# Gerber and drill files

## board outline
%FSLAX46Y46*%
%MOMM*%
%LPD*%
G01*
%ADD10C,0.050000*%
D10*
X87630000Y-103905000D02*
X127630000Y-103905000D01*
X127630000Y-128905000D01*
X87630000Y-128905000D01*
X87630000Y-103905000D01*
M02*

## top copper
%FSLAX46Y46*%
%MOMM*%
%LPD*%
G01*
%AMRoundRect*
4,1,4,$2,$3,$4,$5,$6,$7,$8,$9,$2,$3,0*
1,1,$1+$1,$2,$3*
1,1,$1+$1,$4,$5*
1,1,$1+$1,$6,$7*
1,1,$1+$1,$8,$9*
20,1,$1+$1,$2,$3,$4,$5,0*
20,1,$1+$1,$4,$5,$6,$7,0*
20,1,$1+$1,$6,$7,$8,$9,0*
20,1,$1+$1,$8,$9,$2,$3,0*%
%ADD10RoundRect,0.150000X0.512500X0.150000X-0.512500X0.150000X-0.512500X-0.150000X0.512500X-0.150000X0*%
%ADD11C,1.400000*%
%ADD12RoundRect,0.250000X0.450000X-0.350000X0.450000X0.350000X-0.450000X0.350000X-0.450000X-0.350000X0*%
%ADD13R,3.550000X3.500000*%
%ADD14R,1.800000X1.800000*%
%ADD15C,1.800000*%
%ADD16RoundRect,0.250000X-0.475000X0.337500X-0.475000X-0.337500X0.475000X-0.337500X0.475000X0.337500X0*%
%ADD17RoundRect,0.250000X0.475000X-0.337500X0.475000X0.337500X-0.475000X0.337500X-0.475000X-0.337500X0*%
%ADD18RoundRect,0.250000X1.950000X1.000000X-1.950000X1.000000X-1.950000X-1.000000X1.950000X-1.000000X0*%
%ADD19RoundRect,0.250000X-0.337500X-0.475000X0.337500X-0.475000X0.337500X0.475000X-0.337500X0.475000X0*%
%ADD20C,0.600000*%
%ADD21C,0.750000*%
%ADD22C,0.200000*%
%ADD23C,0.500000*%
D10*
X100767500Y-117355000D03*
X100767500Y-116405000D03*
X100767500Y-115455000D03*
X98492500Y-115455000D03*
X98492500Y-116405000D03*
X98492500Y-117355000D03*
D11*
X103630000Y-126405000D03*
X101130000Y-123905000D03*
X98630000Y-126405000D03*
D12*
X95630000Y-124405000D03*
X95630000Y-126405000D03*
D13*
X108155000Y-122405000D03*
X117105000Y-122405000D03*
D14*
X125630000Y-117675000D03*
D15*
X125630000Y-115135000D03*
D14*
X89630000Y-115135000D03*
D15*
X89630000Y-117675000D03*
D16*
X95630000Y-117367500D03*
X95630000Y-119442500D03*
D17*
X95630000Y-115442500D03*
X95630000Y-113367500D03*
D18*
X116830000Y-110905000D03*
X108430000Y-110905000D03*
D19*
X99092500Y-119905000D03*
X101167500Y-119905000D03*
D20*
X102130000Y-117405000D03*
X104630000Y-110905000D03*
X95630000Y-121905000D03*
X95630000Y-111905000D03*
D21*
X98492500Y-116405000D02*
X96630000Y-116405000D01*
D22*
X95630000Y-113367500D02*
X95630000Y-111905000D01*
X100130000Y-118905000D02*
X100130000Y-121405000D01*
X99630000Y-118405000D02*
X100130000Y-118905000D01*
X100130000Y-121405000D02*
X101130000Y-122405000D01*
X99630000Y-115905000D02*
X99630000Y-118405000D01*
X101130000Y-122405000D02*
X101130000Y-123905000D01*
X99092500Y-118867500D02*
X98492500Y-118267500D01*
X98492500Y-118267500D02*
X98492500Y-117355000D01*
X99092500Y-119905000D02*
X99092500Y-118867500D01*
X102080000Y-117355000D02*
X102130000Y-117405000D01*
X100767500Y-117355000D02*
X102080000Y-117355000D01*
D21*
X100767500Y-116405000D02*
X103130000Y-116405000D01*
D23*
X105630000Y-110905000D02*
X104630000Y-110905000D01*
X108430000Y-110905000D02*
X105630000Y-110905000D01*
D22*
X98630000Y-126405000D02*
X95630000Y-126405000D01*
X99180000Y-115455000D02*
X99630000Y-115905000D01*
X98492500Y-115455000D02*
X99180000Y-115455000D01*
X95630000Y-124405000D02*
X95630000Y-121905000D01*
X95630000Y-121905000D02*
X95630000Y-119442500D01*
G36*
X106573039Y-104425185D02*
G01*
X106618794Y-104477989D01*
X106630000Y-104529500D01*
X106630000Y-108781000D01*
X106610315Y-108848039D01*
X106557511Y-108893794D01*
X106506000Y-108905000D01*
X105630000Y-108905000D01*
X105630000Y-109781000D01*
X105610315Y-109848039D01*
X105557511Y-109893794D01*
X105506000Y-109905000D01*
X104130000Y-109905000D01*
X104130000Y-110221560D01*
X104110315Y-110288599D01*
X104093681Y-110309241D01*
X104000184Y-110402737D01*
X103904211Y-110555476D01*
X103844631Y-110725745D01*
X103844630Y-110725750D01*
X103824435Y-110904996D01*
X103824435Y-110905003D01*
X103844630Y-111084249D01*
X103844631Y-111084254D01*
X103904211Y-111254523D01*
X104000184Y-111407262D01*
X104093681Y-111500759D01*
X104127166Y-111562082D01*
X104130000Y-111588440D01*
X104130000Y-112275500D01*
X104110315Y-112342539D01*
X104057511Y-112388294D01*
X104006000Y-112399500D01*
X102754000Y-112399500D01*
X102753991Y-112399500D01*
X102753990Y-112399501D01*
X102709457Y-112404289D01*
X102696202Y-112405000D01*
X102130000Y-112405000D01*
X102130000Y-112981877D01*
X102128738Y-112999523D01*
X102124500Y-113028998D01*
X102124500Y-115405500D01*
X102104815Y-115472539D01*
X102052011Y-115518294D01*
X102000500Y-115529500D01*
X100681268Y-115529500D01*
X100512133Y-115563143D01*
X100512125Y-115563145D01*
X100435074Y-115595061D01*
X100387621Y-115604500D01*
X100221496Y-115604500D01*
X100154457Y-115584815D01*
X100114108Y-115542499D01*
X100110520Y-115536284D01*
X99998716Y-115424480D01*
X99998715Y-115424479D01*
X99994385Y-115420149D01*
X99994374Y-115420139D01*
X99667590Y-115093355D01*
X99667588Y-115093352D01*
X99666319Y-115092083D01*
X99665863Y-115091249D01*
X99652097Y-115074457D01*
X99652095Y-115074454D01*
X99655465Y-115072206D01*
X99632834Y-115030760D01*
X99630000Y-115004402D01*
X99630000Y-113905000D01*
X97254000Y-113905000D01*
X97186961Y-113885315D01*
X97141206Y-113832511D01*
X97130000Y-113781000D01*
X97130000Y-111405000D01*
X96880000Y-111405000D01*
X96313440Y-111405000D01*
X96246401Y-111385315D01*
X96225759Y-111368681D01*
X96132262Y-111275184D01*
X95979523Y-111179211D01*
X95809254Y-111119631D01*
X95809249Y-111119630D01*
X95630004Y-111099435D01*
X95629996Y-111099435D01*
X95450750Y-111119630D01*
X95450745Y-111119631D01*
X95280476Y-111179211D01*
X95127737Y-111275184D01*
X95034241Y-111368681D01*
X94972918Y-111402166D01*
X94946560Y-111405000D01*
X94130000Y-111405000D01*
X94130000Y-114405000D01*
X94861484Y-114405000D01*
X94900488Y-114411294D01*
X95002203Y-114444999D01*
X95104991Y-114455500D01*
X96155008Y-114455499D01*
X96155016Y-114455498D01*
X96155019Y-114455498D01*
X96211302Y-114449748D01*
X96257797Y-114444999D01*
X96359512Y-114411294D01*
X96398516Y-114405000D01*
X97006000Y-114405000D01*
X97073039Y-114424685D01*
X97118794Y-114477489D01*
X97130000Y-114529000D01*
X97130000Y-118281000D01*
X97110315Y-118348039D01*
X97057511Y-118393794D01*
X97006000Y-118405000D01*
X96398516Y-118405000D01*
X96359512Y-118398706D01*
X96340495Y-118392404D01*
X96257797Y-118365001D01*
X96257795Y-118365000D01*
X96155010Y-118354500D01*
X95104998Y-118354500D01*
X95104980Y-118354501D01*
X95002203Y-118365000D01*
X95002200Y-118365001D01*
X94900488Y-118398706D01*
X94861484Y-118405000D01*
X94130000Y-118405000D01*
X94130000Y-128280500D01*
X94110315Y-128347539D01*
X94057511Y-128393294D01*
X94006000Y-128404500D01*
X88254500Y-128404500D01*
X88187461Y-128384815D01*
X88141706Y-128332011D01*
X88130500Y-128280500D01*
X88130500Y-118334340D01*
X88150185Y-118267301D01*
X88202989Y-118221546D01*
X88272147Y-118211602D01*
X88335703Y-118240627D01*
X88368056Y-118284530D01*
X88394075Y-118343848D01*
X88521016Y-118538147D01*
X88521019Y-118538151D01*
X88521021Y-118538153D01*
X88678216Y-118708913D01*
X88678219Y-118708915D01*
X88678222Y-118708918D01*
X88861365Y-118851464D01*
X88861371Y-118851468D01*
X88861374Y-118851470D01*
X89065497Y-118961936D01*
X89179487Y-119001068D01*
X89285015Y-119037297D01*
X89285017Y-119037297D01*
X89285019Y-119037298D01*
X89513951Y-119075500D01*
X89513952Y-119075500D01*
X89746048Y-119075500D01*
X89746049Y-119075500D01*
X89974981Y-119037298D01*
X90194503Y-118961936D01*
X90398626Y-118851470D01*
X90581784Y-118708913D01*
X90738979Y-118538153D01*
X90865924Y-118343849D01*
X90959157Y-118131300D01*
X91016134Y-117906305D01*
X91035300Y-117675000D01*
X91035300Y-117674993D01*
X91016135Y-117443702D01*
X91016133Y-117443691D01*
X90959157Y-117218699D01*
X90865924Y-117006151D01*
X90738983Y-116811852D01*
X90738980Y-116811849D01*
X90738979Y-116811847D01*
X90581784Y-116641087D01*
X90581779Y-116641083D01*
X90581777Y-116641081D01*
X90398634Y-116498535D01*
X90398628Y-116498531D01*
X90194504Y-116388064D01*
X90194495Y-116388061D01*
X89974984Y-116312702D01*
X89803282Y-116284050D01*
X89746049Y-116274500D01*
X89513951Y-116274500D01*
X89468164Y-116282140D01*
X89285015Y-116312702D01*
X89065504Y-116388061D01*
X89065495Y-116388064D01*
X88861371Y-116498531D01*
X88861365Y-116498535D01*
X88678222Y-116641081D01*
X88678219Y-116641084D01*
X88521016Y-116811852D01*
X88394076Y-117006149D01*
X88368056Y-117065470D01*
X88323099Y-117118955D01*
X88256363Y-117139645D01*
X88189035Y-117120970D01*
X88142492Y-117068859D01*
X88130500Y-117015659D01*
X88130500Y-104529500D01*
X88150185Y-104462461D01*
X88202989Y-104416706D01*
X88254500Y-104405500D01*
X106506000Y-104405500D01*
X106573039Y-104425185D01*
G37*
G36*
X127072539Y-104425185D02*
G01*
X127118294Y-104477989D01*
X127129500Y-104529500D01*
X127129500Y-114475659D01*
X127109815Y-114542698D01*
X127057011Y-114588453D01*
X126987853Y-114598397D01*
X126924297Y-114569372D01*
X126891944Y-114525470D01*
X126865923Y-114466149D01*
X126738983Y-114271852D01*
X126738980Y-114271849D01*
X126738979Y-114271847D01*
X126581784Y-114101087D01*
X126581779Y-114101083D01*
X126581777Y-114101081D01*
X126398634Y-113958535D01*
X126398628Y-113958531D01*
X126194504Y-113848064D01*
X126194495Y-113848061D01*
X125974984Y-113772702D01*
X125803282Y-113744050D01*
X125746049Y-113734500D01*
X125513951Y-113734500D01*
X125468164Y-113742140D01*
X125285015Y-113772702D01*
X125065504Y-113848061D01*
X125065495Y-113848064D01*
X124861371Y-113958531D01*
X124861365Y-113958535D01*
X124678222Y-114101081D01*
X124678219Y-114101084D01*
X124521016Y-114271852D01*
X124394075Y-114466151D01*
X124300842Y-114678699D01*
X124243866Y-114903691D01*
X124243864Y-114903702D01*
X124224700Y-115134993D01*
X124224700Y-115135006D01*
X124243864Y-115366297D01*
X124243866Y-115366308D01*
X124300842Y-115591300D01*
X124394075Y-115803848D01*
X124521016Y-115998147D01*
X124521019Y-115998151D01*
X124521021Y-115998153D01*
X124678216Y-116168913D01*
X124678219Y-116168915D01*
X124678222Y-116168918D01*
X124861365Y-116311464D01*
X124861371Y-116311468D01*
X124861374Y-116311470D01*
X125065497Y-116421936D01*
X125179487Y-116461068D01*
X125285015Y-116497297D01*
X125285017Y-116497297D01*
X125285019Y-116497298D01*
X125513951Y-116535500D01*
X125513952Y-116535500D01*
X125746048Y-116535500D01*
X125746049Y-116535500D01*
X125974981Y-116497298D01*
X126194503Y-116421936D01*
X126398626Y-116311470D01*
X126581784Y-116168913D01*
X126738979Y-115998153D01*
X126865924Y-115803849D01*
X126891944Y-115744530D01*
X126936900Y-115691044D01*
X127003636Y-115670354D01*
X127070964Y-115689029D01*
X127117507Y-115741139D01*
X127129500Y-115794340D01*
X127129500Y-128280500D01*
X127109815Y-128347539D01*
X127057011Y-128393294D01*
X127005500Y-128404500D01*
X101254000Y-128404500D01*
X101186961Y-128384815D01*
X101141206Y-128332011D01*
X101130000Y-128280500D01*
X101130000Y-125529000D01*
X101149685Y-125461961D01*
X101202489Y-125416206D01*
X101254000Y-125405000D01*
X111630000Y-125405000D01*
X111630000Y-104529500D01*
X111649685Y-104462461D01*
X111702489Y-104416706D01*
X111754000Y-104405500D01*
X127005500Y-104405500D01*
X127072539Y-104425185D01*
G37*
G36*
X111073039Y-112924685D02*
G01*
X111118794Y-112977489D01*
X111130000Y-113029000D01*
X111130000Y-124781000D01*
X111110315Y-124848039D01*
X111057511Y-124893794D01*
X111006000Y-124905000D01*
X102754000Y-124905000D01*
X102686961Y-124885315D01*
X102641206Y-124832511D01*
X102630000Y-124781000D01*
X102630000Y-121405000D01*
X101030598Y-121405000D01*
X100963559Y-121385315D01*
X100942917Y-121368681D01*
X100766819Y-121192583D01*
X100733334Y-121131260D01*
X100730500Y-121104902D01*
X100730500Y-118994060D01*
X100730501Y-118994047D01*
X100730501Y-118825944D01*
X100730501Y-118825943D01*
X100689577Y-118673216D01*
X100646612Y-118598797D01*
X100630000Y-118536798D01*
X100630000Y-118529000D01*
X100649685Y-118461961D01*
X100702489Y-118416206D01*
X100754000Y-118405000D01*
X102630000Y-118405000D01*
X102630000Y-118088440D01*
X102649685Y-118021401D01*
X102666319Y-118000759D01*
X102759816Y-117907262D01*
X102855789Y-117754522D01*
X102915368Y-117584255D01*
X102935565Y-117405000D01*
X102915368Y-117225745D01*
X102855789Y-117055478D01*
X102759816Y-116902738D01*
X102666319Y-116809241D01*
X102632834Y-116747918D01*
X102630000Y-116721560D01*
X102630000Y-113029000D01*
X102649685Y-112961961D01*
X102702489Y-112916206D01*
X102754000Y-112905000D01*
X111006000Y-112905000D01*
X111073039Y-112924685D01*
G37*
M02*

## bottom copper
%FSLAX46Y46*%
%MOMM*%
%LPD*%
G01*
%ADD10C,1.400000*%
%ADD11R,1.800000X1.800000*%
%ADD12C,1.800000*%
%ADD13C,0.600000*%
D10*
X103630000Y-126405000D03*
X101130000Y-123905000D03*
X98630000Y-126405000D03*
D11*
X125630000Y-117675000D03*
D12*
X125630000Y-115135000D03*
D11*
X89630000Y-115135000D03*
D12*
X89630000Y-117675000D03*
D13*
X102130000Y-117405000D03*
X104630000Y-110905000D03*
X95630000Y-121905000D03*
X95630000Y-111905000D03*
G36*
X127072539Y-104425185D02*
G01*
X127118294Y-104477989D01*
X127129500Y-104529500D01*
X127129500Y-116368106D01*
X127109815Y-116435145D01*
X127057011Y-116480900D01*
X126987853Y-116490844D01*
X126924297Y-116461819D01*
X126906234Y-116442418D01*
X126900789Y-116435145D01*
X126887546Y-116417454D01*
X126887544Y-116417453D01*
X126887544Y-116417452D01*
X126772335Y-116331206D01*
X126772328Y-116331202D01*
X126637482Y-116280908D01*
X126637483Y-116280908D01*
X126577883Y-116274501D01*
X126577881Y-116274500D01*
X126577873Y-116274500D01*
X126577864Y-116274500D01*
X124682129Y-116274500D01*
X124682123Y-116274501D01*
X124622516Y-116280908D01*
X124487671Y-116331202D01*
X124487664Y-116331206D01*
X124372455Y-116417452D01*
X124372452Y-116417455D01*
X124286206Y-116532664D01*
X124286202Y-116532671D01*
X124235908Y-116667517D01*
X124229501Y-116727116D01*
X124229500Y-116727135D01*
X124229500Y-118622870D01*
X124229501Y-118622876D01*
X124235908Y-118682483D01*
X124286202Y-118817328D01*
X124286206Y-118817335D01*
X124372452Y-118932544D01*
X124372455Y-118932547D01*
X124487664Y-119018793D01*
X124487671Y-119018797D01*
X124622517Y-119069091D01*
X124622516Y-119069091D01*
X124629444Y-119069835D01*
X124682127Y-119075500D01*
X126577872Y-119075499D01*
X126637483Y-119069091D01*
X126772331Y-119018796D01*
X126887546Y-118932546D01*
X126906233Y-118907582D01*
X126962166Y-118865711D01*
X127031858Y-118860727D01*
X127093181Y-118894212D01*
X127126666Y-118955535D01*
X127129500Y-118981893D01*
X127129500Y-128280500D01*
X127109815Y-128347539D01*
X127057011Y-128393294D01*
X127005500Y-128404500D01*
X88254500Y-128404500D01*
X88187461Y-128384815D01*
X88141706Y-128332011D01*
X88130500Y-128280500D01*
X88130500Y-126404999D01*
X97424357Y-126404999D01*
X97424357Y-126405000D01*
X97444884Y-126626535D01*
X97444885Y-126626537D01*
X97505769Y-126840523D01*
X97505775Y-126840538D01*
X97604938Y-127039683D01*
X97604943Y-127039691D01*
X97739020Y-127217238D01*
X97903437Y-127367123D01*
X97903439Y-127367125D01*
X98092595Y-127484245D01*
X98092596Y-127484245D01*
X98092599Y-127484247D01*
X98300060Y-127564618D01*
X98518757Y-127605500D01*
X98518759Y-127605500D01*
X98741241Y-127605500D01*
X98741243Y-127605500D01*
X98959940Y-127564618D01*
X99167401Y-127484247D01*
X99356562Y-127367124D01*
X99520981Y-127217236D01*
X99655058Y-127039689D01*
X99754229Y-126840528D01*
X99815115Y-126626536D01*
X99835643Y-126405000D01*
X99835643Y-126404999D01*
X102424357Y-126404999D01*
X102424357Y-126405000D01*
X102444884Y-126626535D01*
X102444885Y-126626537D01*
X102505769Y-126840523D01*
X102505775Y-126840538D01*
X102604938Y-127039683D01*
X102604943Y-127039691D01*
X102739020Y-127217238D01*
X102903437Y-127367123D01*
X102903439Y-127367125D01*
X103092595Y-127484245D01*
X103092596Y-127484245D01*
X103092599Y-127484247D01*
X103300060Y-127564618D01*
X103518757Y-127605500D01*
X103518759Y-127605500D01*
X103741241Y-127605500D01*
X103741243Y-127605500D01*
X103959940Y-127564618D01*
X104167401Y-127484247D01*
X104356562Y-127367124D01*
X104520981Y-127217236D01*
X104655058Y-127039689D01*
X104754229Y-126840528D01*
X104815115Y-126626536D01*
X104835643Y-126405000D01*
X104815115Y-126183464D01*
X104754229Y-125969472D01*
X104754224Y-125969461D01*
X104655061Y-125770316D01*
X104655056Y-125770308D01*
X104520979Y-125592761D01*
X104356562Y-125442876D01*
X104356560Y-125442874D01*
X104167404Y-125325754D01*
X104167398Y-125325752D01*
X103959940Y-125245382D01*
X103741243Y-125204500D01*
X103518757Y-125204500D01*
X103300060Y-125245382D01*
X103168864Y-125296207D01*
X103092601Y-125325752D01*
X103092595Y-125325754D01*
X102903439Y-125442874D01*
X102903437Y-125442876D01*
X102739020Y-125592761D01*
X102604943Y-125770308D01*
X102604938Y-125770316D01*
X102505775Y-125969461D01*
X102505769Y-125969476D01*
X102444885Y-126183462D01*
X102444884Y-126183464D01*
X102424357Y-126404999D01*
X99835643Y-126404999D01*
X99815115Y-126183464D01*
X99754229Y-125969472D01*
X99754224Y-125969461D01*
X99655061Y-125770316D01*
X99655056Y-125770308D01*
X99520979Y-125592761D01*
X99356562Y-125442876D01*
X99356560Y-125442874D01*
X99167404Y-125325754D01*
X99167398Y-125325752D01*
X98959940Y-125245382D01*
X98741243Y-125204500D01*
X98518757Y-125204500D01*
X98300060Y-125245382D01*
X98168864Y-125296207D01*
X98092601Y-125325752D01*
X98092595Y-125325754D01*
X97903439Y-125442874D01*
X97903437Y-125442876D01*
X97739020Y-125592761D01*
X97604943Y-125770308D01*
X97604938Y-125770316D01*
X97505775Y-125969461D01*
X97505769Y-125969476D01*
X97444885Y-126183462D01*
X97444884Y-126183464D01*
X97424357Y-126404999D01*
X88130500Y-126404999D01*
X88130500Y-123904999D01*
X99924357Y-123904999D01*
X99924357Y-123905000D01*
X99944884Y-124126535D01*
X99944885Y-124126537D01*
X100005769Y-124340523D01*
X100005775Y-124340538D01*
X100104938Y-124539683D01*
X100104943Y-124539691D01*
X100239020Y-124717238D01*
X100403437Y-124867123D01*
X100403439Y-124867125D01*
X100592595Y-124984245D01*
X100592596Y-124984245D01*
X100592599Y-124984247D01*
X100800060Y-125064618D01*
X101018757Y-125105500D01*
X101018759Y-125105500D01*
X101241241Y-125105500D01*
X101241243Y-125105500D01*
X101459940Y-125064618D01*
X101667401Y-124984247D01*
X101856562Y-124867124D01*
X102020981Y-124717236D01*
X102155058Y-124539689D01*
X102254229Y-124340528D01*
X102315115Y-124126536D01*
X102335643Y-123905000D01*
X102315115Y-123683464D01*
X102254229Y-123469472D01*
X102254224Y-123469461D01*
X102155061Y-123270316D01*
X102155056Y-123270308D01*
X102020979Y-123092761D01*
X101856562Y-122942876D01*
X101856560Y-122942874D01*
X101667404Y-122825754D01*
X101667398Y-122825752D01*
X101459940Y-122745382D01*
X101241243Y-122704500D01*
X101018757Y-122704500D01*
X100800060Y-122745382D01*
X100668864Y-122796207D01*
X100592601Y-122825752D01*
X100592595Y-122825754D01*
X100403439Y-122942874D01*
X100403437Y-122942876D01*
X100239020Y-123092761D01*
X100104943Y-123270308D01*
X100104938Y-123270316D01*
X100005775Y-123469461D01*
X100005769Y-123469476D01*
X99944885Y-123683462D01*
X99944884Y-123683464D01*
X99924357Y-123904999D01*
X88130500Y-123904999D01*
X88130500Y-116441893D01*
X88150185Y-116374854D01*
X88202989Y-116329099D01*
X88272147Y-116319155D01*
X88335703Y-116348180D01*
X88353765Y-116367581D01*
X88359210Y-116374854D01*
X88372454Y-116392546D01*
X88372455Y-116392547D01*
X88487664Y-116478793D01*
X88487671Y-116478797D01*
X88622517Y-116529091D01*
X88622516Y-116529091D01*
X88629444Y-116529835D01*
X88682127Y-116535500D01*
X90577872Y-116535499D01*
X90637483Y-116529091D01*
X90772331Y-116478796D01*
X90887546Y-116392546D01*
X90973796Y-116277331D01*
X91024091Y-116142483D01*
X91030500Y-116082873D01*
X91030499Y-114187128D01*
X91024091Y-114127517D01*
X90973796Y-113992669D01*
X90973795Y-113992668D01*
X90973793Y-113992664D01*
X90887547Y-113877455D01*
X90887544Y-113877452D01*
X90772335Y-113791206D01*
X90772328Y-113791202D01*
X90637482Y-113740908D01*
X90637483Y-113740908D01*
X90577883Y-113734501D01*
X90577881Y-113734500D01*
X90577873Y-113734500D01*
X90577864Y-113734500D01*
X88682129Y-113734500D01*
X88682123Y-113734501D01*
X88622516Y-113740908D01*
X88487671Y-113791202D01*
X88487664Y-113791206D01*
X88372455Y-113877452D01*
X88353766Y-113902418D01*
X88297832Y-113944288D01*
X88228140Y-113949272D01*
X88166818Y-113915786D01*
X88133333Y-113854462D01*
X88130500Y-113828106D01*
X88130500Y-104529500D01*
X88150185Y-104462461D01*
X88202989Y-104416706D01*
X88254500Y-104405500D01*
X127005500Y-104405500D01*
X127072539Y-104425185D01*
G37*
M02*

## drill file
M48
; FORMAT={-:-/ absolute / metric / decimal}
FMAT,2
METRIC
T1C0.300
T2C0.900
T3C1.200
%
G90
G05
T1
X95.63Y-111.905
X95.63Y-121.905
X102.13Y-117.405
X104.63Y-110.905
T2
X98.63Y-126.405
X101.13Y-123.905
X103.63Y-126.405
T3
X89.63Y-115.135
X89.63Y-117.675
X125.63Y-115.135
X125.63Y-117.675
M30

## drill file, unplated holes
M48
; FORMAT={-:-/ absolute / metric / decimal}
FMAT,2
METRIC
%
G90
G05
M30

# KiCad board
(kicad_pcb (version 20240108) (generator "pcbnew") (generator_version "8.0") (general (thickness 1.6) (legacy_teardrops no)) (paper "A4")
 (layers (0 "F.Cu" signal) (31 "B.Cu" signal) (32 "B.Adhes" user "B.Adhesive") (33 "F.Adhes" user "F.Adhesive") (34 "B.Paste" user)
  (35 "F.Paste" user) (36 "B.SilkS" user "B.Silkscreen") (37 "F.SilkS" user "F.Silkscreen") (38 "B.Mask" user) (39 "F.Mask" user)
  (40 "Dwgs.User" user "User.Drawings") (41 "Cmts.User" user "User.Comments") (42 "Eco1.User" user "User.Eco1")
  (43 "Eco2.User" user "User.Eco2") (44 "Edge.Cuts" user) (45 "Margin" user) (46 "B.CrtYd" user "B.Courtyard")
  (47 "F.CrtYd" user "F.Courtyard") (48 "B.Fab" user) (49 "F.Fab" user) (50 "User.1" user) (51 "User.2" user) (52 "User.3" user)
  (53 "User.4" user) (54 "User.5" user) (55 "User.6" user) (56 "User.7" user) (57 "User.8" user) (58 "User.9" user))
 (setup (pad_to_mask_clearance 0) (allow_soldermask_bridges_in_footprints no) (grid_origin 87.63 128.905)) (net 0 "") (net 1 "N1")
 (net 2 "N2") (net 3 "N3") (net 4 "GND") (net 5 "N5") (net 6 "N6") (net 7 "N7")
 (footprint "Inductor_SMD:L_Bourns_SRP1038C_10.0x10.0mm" (layer "F.Cu") (at 112.63 122.405)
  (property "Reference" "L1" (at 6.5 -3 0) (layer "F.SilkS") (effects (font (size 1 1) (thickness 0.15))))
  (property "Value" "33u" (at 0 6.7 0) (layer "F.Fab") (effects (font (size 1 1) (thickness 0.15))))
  (pad "1" smd rect (at -4.475 0) (size 3.55 3.5) (layers "F.Cu" "F.Paste" "F.Mask") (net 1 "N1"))
  (pad "2" smd rect (at 4.475 0) (size 3.55 3.5) (layers "F.Cu" "F.Paste" "F.Mask") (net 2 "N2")))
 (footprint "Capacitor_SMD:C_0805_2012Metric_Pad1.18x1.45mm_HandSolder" (layer "F.Cu") (at 95.63 118.405 -90)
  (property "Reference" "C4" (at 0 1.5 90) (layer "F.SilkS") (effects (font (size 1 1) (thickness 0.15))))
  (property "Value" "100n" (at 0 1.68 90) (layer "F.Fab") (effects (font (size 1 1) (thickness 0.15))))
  (pad "1" smd roundrect (at -1.0375 0 270) (size 1.175 1.45) (layers "F.Cu" "F.Paste" "F.Mask") (roundrect_rratio 0.212766) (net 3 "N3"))
  (pad "2" smd roundrect (at 1.0375 0 270) (size 1.175 1.45) (layers "F.Cu" "F.Paste" "F.Mask") (roundrect_rratio 0.212766) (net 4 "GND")))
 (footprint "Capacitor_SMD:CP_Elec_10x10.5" (layer "F.Cu") (at 112.63 110.905 180)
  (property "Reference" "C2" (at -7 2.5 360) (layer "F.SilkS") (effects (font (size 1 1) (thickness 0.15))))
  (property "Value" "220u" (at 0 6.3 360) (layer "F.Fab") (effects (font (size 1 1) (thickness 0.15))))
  (pad "1" smd roundrect (at -4.2 0 180) (size 4.4 2.5) (layers "F.Cu" "F.Paste" "F.Mask") (roundrect_rratio 0.1) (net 2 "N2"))
  (pad "2" smd roundrect (at 4.2 0 180) (size 4.4 2.5) (layers "F.Cu" "F.Paste" "F.Mask") (roundrect_rratio 0.1) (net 4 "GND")))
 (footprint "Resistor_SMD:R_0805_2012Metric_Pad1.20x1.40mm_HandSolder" (layer "F.Cu") (at 95.63 125.405 90)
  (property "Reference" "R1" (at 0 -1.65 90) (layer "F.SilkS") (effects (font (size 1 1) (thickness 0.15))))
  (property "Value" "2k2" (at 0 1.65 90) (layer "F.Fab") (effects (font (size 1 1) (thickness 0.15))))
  (pad "1" smd roundrect (at -1 0 90) (size 1.2 1.4) (layers "F.Cu" "F.Paste" "F.Mask") (roundrect_rratio 0.208333) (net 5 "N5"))
  (pad "2" smd roundrect (at 1 0 90) (size 1.2 1.4) (layers "F.Cu" "F.Paste" "F.Mask") (roundrect_rratio 0.208333) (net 4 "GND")))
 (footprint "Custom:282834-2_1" (layer "F.Cu") (at 89.63 115.135 -90)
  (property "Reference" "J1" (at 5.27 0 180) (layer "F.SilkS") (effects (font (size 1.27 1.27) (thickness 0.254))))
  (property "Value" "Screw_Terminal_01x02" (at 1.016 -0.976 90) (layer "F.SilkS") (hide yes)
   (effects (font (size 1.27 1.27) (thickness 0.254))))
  (pad "1" thru_hole rect (at 0 0 270) (size 1.8 1.8) (drill 1.2) (layers "*.Cu" "*.Mask") (remove_unused_layers no) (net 3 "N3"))
  (pad "2" thru_hole circle (at 2.54 0 270) (size 1.8 1.8) (drill 1.2) (layers "*.Cu" "*.Mask") (remove_unused_layers no) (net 4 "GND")))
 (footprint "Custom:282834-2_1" (layer "F.Cu") (at 125.63 117.675 90)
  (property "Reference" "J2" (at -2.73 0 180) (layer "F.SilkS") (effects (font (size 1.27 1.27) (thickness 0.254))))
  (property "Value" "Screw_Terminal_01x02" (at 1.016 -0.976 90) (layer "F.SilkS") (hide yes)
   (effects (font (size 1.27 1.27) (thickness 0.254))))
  (pad "1" thru_hole rect (at 0 0 90) (size 1.8 1.8) (drill 1.2) (layers "*.Cu" "*.Mask") (remove_unused_layers no) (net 2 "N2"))
  (pad "2" thru_hole circle (at 2.54 0 90) (size 1.8 1.8) (drill 1.2) (layers "*.Cu" "*.Mask") (remove_unused_layers no) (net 4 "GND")))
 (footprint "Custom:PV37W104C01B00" (layer "F.Cu") (at 98.63 126.405)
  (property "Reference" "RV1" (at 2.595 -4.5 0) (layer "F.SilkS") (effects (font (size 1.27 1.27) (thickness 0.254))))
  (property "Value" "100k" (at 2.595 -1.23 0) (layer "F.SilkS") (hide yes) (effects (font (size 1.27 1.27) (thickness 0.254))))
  (pad "1" thru_hole circle (at 0 0) (size 1.4 1.4) (drill 0.9) (layers "*.Cu" "*.Mask") (remove_unused_layers no) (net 5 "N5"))
  (pad "2" thru_hole circle (at 2.5 -2.5) (size 1.4 1.4) (drill 0.9) (layers "*.Cu" "*.Mask") (remove_unused_layers no) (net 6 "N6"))
  (pad "3" thru_hole circle (at 5 0) (size 1.4 1.4) (drill 0.9) (layers "*.Cu" "*.Mask") (remove_unused_layers no) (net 2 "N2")))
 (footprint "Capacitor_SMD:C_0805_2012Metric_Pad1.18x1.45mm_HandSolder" (layer "F.Cu") (at 100.13 119.905)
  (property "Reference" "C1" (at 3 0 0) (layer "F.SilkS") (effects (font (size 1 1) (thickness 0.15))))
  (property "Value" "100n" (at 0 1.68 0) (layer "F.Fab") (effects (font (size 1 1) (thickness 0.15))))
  (pad "1" smd roundrect (at -1.0375 0) (size 1.175 1.45) (layers "F.Cu" "F.Paste" "F.Mask") (roundrect_rratio 0.212766) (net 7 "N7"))
  (pad "2" smd roundrect (at 1.0375 0) (size 1.175 1.45) (layers "F.Cu" "F.Paste" "F.Mask") (roundrect_rratio 0.212766) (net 1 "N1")))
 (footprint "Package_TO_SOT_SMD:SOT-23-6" (layer "F.Cu") (at 99.63 116.405 180)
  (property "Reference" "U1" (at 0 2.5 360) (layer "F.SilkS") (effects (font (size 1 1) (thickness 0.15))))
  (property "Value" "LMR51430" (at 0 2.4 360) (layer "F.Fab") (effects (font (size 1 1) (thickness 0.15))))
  (pad "1" smd roundrect (at -1.1375 -0.95 180) (size 1.325 0.6) (layers "F.Cu" "F.Paste" "F.Mask") (roundrect_rratio 0.25) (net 4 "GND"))
  (pad "2" smd roundrect (at -1.1375 0 180) (size 1.325 0.6) (layers "F.Cu" "F.Paste" "F.Mask") (roundrect_rratio 0.25) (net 1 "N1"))
  (pad "3" smd roundrect (at -1.1375 0.95 180) (size 1.325 0.6) (layers "F.Cu" "F.Paste" "F.Mask") (roundrect_rratio 0.25) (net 3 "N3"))
  (pad "4" smd roundrect (at 1.1375 0.95 180) (size 1.325 0.6) (layers "F.Cu" "F.Paste" "F.Mask") (roundrect_rratio 0.25) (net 6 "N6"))
  (pad "5" smd roundrect (at 1.1375 0 180) (size 1.325 0.6) (layers "F.Cu" "F.Paste" "F.Mask") (roundrect_rratio 0.25) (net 3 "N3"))
  (pad "6" smd roundrect (at 1.1375 -0.95 180) (size 1.325 0.6) (layers "F.Cu" "F.Paste" "F.Mask") (roundrect_rratio 0.25) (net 7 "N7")))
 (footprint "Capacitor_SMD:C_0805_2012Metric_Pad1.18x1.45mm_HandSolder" (layer "F.Cu") (at 95.63 114.405 90)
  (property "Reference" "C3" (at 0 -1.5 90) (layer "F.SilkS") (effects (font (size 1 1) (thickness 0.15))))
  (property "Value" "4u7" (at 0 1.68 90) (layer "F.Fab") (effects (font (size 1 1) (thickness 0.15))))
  (pad "1" smd roundrect (at -1.0375 0 90) (size 1.175 1.45) (layers "F.Cu" "F.Paste" "F.Mask") (roundrect_rratio 0.212766) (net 3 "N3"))
  (pad "2" smd roundrect (at 1.0375 0 90) (size 1.175 1.45) (layers "F.Cu" "F.Paste" "F.Mask") (roundrect_rratio 0.212766) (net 4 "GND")))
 (gr_rect (start 87.63 103.905) (end 127.63 128.905) (stroke (width 0.05) (type default)) (fill none) (layer "Edge.Cuts"))
 (segment (start 99.0925 118.8675) (end 98.4925 118.2675) (width 0.2) (layer "F.Cu") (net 7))
 (segment (start 98.4925 118.2675) (end 98.4925 117.355) (width 0.2) (layer "F.Cu") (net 7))
 (segment (start 99.0925 119.905) (end 99.0925 118.8675) (width 0.2) (layer "F.Cu") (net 7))
 (segment (start 100.7675 116.405) (end 103.13 116.405) (width 0.75) (layer "F.Cu") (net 1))
 (segment (start 108.43 110.905) (end 105.63 110.905) (width 0.5) (layer "F.Cu") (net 4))
 (segment (start 95.63 121.905) (end 95.63 119.4425) (width 0.2) (layer "F.Cu") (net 4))
 (segment (start 102.08 117.355) (end 102.13 117.405) (width 0.2) (layer "F.Cu") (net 4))
 (segment (start 95.63 113.3675) (end 95.63 111.905) (width 0.2) (layer "F.Cu") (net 4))
 (segment (start 100.7675 117.355) (end 102.08 117.355) (width 0.2) (layer "F.Cu") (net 4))
 (segment (start 105.63 110.905) (end 104.63 110.905) (width 0.5) (layer "F.Cu") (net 4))
 (segment (start 95.63 124.405) (end 95.63 121.905) (width 0.2) (layer "F.Cu") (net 4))
 (via (at 95.63 111.905) (size 0.6) (drill 0.3) (layers "F.Cu" "B.Cu") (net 4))
 (via (at 104.63 110.905) (size 0.6) (drill 0.3) (layers "F.Cu" "B.Cu") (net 4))
 (via (at 95.63 121.905) (size 0.6) (drill 0.3) (layers "F.Cu" "B.Cu") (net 4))
 (via (at 102.13 117.405) (size 0.6) (drill 0.3) (layers "F.Cu" "B.Cu") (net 4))
 (segment (start 98.4925 116.405) (end 96.63 116.405) (width 0.75) (layer "F.Cu") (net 3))
 (segment (start 98.63 126.405) (end 95.63 126.405) (width 0.2) (layer "F.Cu") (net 5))
 (segment (start 99.63 118.405) (end 100.13 118.905) (width 0.2) (layer "F.Cu") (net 6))
 (segment (start 100.13 121.405) (end 101.13 122.405) (width 0.2) (layer "F.Cu") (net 6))
 (segment (start 98.4925 115.455) (end 99.18 115.455) (width 0.2) (layer "F.Cu") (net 6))
 (segment (start 99.18 115.455) (end 99.63 115.905) (width 0.2) (layer "F.Cu") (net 6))
 (segment (start 101.13 122.405) (end 101.13 123.905) (width 0.2) (layer "F.Cu") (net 6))
 (segment (start 99.63 115.905) (end 99.63 118.405) (width 0.2) (layer "F.Cu") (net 6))
 (segment (start 100.13 118.905) (end 100.13 121.405) (width 0.2) (layer "F.Cu") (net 6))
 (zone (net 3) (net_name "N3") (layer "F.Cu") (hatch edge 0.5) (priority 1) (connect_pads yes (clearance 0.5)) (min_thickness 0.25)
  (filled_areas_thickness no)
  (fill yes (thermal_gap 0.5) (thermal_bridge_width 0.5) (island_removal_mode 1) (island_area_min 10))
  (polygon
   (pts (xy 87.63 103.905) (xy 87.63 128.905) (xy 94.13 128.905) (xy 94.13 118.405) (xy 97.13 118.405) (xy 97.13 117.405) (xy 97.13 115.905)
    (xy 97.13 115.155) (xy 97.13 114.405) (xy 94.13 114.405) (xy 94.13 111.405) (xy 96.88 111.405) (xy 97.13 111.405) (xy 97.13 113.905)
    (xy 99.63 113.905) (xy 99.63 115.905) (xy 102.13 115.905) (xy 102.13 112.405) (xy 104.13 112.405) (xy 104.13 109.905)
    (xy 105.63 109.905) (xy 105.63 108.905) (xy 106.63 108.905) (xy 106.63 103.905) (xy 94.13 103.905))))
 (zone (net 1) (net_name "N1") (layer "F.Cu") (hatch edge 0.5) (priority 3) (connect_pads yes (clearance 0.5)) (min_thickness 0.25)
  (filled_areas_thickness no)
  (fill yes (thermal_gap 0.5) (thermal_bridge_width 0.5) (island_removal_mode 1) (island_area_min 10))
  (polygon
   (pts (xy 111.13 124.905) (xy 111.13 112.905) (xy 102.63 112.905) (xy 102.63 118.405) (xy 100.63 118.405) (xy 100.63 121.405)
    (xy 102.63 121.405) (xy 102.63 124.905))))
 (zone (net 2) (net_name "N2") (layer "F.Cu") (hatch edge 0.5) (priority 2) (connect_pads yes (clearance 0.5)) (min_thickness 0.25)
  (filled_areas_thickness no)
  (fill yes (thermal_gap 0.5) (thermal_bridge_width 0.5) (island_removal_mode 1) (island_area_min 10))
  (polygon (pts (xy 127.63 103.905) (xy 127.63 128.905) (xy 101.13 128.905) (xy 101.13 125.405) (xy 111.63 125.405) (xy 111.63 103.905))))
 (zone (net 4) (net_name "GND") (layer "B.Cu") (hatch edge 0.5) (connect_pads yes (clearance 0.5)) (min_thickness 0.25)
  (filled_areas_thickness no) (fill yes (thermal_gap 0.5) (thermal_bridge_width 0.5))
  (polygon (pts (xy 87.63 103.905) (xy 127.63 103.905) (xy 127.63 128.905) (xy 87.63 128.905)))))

